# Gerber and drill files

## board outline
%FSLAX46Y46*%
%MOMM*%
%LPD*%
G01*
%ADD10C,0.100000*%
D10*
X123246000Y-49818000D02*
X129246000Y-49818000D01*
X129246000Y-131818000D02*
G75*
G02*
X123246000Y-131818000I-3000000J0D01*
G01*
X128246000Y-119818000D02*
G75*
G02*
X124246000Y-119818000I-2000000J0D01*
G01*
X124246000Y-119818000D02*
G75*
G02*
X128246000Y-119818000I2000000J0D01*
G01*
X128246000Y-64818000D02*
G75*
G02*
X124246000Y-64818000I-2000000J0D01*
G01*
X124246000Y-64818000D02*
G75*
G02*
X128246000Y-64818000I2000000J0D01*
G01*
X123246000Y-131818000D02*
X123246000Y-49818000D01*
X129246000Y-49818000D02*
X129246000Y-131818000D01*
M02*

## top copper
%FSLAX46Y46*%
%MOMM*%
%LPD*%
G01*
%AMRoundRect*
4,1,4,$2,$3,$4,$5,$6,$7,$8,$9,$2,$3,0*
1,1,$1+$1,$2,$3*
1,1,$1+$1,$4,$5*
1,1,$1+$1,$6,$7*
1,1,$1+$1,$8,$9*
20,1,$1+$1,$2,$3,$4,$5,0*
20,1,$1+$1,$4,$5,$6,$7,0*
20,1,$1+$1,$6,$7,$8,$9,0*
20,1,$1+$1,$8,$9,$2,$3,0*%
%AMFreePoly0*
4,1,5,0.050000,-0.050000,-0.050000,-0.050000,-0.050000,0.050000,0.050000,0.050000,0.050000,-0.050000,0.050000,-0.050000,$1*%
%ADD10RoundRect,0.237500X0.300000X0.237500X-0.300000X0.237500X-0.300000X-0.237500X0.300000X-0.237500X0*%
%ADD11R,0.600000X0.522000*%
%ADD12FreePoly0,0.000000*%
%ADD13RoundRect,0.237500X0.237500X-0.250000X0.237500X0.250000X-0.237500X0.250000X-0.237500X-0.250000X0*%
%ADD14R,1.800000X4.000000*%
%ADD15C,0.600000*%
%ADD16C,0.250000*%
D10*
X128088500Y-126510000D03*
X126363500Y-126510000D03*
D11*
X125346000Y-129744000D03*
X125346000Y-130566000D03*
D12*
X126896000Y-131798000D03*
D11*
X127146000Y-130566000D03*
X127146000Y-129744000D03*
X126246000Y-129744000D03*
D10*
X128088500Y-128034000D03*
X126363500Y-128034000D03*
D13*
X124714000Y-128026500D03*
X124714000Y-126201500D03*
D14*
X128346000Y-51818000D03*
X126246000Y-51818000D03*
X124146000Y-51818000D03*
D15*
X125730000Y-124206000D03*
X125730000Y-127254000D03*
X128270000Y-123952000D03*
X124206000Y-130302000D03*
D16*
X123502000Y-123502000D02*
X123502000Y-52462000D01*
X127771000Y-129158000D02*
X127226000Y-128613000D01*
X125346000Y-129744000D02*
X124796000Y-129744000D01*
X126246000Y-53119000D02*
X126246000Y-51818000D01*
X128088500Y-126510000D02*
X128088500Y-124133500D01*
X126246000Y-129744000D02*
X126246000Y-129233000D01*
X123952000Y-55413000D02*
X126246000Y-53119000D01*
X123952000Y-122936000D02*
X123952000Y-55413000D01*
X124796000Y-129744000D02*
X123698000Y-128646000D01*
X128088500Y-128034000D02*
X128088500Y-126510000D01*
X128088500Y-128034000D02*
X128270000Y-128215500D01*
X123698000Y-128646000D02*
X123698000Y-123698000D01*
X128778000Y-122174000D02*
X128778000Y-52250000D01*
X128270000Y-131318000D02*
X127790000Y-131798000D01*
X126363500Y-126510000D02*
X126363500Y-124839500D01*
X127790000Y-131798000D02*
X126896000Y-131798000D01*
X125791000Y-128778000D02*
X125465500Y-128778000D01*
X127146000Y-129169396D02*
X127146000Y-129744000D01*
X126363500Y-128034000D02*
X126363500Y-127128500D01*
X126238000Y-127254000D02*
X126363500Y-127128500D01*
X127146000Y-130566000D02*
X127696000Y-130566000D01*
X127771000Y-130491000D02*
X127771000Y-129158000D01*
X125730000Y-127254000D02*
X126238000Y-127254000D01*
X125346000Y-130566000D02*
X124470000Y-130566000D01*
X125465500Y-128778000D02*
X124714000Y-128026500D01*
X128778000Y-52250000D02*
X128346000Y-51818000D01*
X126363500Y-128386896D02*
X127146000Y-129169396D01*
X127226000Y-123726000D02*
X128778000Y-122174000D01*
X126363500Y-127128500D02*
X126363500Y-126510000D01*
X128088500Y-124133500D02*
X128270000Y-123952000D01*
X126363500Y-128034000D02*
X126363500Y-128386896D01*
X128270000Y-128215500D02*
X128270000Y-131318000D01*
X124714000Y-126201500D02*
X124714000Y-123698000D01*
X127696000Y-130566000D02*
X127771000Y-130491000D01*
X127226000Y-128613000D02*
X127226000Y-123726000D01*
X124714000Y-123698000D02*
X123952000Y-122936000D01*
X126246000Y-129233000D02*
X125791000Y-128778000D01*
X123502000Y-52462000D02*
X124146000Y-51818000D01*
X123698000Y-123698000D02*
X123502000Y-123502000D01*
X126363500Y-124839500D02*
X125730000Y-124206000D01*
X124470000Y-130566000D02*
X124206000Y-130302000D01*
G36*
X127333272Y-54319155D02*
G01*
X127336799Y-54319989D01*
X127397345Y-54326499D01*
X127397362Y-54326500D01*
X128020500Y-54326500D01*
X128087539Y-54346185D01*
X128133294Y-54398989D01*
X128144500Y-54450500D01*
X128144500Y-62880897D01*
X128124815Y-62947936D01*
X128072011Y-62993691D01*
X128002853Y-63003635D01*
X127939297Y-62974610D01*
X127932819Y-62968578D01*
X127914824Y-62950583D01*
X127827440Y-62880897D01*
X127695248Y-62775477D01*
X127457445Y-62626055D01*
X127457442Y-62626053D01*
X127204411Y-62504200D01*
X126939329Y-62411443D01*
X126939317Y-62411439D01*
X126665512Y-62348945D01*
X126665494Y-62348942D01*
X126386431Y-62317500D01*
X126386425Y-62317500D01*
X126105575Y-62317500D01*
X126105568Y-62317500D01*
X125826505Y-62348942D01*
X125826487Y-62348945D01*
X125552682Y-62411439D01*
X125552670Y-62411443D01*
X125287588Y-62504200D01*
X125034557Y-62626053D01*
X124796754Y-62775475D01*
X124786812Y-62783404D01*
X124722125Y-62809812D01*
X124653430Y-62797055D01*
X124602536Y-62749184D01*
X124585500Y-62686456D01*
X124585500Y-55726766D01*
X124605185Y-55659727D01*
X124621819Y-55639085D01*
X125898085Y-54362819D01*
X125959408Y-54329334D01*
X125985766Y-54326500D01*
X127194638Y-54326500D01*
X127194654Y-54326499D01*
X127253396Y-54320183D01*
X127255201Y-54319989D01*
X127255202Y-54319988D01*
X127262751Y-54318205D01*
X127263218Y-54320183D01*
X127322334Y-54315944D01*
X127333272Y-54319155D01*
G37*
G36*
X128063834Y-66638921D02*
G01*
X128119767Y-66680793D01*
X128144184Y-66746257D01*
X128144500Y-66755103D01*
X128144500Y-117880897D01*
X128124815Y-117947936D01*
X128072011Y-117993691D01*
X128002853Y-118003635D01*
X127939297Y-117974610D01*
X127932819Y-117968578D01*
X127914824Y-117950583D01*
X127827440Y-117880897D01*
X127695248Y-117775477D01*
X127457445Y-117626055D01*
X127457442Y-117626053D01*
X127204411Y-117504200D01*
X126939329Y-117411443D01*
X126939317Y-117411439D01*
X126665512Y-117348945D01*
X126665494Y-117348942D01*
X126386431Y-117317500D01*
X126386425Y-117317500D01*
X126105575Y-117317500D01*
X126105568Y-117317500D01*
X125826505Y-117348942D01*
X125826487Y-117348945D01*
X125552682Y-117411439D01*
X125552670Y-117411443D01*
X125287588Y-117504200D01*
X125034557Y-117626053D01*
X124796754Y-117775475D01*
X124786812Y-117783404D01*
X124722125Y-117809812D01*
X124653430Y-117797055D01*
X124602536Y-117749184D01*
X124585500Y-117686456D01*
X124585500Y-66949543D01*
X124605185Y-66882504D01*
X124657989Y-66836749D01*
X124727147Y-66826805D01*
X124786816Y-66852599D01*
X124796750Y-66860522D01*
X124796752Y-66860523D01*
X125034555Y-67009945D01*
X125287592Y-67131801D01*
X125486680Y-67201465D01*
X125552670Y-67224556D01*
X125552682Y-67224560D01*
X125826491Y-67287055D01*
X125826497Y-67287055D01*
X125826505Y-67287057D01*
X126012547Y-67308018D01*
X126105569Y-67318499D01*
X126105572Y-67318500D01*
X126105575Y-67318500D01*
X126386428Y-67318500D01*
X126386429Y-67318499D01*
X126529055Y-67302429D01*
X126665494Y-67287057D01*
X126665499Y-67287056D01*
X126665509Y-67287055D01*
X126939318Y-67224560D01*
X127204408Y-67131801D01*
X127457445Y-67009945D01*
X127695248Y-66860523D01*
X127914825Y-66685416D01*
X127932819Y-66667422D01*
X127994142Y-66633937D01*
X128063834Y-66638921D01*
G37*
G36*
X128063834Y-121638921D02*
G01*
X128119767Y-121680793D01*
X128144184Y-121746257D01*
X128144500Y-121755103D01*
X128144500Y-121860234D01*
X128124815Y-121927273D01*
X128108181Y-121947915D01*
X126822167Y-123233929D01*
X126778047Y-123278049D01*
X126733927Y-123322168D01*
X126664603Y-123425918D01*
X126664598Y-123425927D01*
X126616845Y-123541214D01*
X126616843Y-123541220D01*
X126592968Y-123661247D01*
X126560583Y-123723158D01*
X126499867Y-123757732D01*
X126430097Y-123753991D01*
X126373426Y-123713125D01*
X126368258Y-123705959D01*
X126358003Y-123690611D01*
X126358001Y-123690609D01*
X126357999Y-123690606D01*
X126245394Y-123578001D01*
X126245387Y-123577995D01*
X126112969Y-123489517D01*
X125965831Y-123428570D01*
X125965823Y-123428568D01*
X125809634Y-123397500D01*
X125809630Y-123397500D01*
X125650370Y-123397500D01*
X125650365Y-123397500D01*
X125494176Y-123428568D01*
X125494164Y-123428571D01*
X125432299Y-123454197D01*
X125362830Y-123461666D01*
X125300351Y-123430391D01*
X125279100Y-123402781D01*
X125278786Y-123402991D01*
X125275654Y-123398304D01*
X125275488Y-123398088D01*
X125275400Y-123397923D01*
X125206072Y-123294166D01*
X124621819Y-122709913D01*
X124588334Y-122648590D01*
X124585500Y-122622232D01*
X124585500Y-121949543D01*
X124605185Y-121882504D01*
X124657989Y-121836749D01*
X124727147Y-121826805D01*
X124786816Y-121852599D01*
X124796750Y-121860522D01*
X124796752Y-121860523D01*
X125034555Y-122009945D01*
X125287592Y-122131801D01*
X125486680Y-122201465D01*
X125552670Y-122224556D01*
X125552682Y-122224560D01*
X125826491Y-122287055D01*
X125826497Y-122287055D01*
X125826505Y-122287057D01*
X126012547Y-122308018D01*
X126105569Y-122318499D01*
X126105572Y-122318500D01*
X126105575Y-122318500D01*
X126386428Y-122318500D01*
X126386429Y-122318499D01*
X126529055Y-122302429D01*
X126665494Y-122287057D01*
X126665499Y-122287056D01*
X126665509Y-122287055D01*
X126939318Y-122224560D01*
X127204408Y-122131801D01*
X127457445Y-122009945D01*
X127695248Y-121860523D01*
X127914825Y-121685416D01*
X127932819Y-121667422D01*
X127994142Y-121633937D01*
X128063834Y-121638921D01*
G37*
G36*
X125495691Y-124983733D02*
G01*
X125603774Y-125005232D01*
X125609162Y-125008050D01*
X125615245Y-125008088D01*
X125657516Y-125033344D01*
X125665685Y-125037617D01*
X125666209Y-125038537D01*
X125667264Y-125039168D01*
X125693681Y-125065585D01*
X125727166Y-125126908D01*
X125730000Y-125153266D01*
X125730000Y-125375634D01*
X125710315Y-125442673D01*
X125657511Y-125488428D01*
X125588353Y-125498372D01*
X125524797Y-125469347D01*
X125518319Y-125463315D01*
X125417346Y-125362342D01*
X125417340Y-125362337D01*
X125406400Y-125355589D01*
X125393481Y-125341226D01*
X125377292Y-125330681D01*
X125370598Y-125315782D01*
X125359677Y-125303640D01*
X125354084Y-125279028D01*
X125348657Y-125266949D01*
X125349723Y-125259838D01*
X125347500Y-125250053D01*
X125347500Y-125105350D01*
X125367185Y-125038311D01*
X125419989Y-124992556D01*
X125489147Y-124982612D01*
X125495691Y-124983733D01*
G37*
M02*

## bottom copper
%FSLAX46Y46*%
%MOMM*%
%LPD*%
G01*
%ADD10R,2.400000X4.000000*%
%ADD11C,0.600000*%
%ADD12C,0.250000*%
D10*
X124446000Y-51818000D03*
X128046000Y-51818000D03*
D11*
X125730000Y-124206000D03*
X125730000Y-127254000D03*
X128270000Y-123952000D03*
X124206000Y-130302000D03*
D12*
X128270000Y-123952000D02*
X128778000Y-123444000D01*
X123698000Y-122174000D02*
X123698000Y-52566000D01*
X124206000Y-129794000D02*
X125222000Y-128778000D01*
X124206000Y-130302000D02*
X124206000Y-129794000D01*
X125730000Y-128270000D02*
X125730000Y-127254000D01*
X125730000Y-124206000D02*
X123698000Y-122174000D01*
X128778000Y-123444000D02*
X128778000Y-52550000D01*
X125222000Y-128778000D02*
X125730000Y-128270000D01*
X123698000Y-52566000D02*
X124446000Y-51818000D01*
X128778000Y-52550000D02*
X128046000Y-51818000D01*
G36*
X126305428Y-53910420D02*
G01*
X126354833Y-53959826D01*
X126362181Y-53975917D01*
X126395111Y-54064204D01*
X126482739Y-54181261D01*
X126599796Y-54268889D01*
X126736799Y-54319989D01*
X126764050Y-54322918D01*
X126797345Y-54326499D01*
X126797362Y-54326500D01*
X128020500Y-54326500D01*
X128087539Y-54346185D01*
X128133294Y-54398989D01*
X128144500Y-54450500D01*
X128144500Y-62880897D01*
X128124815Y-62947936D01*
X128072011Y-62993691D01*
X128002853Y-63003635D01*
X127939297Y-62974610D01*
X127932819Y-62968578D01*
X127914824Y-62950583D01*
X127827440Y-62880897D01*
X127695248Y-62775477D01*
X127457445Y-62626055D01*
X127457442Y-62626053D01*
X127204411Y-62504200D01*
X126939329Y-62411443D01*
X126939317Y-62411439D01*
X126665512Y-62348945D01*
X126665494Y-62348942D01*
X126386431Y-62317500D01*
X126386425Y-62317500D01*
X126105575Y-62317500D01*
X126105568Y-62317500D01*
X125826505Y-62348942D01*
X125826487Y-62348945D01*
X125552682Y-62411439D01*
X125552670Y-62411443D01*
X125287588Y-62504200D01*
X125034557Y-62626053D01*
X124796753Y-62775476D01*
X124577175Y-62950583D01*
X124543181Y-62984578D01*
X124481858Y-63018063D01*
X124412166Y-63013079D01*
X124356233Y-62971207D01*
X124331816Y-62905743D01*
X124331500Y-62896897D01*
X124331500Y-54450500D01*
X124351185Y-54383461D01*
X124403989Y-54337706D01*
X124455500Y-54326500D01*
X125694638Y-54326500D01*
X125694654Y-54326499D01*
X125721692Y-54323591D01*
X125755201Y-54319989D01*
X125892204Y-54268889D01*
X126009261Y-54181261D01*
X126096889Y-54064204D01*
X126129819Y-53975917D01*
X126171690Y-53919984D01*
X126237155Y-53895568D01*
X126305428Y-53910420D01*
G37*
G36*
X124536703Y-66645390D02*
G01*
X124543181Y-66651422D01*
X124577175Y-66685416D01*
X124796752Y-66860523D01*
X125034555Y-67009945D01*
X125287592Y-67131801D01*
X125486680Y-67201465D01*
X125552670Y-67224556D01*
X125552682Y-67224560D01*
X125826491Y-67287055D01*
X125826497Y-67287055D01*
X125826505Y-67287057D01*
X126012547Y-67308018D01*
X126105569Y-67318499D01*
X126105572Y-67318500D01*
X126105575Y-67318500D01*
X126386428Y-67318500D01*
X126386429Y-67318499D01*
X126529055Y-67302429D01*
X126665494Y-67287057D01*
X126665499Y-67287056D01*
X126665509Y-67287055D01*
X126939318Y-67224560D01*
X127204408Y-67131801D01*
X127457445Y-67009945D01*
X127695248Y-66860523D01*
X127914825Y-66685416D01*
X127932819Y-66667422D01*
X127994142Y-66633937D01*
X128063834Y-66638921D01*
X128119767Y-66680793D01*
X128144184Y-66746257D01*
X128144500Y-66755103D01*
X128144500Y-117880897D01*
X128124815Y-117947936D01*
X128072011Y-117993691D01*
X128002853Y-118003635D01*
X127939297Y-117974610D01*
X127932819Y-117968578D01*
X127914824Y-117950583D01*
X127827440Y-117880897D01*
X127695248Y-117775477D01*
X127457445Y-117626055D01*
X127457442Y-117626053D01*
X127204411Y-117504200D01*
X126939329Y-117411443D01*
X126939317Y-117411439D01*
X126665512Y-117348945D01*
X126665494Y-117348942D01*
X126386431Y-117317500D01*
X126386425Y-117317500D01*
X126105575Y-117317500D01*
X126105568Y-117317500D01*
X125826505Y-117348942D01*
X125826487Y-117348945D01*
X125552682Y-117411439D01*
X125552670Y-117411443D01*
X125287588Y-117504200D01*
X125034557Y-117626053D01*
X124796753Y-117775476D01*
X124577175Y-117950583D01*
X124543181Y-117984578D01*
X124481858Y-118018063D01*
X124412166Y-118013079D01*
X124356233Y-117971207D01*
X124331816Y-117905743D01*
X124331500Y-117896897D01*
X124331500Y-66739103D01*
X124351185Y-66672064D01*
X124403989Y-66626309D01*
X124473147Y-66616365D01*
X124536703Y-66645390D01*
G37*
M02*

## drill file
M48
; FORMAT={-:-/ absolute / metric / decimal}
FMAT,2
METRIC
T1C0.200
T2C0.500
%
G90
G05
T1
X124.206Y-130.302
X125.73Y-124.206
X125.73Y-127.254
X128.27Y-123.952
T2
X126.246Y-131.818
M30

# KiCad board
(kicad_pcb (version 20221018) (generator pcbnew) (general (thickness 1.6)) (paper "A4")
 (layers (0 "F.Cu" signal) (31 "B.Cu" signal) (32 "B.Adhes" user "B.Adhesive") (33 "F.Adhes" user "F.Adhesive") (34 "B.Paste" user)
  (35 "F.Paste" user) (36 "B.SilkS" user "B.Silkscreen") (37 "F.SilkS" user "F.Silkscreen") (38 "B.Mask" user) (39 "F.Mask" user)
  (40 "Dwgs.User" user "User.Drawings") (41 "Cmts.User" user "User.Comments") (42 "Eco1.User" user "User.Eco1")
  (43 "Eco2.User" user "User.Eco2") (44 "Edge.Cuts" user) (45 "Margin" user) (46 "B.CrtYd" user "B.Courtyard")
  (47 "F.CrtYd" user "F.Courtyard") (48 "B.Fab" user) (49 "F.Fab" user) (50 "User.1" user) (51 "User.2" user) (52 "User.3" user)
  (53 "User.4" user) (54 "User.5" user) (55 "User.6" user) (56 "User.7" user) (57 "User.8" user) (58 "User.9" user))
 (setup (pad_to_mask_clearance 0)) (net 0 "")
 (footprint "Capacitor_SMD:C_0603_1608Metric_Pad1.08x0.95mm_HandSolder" (layer "F.Cu") (at 127.226 126.51 180)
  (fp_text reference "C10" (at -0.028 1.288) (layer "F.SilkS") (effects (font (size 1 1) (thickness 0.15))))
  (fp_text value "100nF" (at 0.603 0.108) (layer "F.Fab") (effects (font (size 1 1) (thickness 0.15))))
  (pad "1" smd roundrect (at -0.8625 0 180) (size 1.075 0.95) (layers "F.Cu" "F.Paste" "F.Mask") (roundrect_rratio 0.25))
  (pad "2" smd roundrect (at 0.8625 0 180) (size 1.075 0.95) (layers "F.Cu" "F.Paste" "F.Mask") (roundrect_rratio 0.25)))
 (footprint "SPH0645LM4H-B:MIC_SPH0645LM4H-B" (layer "F.Cu") (at 126.246 131.818)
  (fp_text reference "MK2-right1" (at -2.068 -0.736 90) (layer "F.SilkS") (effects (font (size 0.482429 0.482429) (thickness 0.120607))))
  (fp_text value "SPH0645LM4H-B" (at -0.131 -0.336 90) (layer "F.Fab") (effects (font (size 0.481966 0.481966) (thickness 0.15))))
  (pad "" np_thru_hole circle (at 0 0) (size 0.5 0.5) (drill 0.5) (layers "*.Cu" "*.Mask"))
  (pad "1" smd rect (at -0.9 -2.074) (size 0.6 0.522) (layers "F.Cu" "F.Paste" "F.Mask"))
  (pad "2" smd rect (at -0.9 -1.252) (size 0.6 0.522) (layers "F.Cu" "F.Paste" "F.Mask"))
  (pad "3" smd custom (at 0.65 -0.02) (size 0.1 0.1) (layers "F.Cu") (zone_connect 0) (thermal_bridge_angle 45)
   (options (clearance outline) (anchor rect)) (primitives))
  (pad "4" smd rect (at 0.9 -1.252) (size 0.6 0.522) (layers "F.Cu" "F.Paste" "F.Mask"))
  (pad "5" smd rect (at 0.9 -2.074) (size 0.6 0.522) (layers "F.Cu" "F.Paste" "F.Mask"))
  (pad "6" smd rect (at 0 -2.074) (size 0.6 0.522) (layers "F.Cu" "F.Paste" "F.Mask")))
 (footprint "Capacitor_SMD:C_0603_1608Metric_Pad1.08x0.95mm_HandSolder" (layer "F.Cu") (at 127.226 128.034 180)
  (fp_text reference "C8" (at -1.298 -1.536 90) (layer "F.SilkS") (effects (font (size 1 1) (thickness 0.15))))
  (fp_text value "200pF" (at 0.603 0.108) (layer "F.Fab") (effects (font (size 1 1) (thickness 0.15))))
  (pad "1" smd roundrect (at -0.8625 0 180) (size 1.075 0.95) (layers "F.Cu" "F.Paste" "F.Mask") (roundrect_rratio 0.25))
  (pad "2" smd roundrect (at 0.8625 0 180) (size 1.075 0.95) (layers "F.Cu" "F.Paste" "F.Mask") (roundrect_rratio 0.25)))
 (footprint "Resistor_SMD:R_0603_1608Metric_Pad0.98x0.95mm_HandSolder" (layer "F.Cu") (at 124.714 127.114 90)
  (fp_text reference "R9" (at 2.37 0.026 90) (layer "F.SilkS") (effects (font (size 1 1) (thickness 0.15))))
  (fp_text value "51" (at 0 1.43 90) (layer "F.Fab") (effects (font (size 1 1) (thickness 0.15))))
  (pad "1" smd roundrect (at -0.9125 0 90) (size 0.975 0.95) (layers "F.Cu" "F.Paste" "F.Mask") (roundrect_rratio 0.25))
  (pad "2" smd roundrect (at 0.9125 0 90) (size 0.975 0.95) (layers "F.Cu" "F.Paste" "F.Mask") (roundrect_rratio 0.25)))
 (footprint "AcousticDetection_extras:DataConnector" (layer "F.Cu") (at 126.246 51.818 -90)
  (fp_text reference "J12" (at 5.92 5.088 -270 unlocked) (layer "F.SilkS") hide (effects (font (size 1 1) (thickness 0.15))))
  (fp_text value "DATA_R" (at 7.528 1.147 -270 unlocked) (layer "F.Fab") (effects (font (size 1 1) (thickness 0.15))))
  (pad "1" smd rect (at 0 -2.1 270) (size 4 1.8) (layers "F.Cu" "F.Paste" "F.Mask") (thermal_bridge_angle 45))
  (pad "2" smd rect (at 0 0 270) (size 4 1.8) (layers "F.Cu" "F.Paste" "F.Mask") (thermal_bridge_angle 45))
  (pad "3" smd rect (at 0 2.1 270) (size 4 1.8) (layers "F.Cu" "F.Paste" "F.Mask") (thermal_bridge_angle 45)))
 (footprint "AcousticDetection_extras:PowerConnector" (layer "B.Cu") (at 126.246 51.818 -90)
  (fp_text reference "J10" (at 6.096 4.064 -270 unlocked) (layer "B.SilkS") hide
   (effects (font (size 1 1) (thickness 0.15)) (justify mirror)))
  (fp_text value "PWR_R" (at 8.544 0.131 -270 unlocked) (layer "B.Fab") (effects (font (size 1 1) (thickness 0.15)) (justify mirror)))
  (pad "1" smd rect (at 0 1.8 270) (size 4 2.4) (layers "B.Cu" "B.Paste" "B.Mask") (thermal_bridge_angle 45))
  (pad "2" smd rect (at 0 -1.8 270) (size 4 2.4) (layers "B.Cu" "B.Paste" "B.Mask") (thermal_bridge_angle 45)))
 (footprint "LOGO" (layer "B.Cu") (at 126.238 132.08 -90)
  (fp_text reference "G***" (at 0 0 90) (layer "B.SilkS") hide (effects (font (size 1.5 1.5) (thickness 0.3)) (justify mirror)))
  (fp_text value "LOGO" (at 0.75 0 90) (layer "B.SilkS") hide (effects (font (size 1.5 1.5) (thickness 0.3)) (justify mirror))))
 (gr_line (start 123.246 49.818) (end 129.246 49.818) (stroke (width 0.1) (type solid)) (layer "Edge.Cuts"))
 (gr_arc (start 129.246 131.818) (mid 126.246 134.818) (end 123.246 131.818) (stroke (width 0.1) (type solid)) (layer "Edge.Cuts"))
 (gr_circle (center 126.246 119.818) (end 126.246 117.818) (stroke (width 0.1) (type default)) (fill none) (layer "Edge.Cuts"))
 (gr_circle (center 126.246 64.818) (end 126.246 62.818) (stroke (width 0.1) (type default)) (fill none) (layer "Edge.Cuts"))
 (gr_line (start 123.246 131.818) (end 123.246 49.818) (stroke (width 0.1) (type solid)) (layer "Edge.Cuts"))
 (gr_line (start 129.246 49.818) (end 129.246 131.818) (stroke (width 0.1) (type solid)) (layer "Edge.Cuts"))
 (segment (start 123.502 123.502) (end 123.502 52.462) (width 0.25) (layer "F.Cu") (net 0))
 (segment (start 127.771 129.158) (end 127.226 128.613) (width 0.25) (layer "F.Cu") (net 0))
 (segment (start 125.346 129.744) (end 124.796 129.744) (width 0.25) (layer "F.Cu") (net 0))
 (segment (start 126.246 53.119) (end 126.246 51.818) (width 0.25) (layer "F.Cu") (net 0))
 (segment (start 128.0885 126.51) (end 128.0885 124.1335) (width 0.25) (layer "F.Cu") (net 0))
 (segment (start 126.246 129.744) (end 126.246 129.233) (width 0.25) (layer "F.Cu") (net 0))
 (segment (start 123.952 55.413) (end 126.246 53.119) (width 0.25) (layer "F.Cu") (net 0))
 (segment (start 123.952 122.936) (end 123.952 55.413) (width 0.25) (layer "F.Cu") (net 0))
 (segment (start 124.796 129.744) (end 123.698 128.646) (width 0.25) (layer "F.Cu") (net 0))
 (segment (start 128.0885 128.034) (end 128.0885 126.51) (width 0.25) (layer "F.Cu") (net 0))
 (segment (start 128.0885 128.034) (end 128.27 128.2155) (width 0.25) (layer "F.Cu") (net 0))
 (segment (start 123.698 128.646) (end 123.698 123.698) (width 0.25) (layer "F.Cu") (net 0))
 (segment (start 128.778 122.174) (end 128.778 52.25) (width 0.25) (layer "F.Cu") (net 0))
 (segment (start 128.27 131.318) (end 127.79 131.798) (width 0.25) (layer "F.Cu") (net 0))
 (segment (start 126.3635 126.51) (end 126.3635 124.8395) (width 0.25) (layer "F.Cu") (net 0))
 (segment (start 127.79 131.798) (end 126.896 131.798) (width 0.25) (layer "F.Cu") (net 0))
 (segment (start 125.791 128.778) (end 125.4655 128.778) (width 0.25) (layer "F.Cu") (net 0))
 (segment (start 127.146 129.169396) (end 127.146 129.744) (width 0.25) (layer "F.Cu") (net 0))
 (segment (start 126.3635 128.034) (end 126.3635 127.1285) (width 0.25) (layer "F.Cu") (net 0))
 (segment (start 126.238 127.254) (end 126.3635 127.1285) (width 0.25) (layer "F.Cu") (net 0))
 (segment (start 127.146 130.566) (end 127.696 130.566) (width 0.25) (layer "F.Cu") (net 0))
 (segment (start 127.771 130.491) (end 127.771 129.158) (width 0.25) (layer "F.Cu") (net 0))
 (segment (start 125.73 127.254) (end 126.238 127.254) (width 0.25) (layer "F.Cu") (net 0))
 (segment (start 125.346 130.566) (end 124.47 130.566) (width 0.25) (layer "F.Cu") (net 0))
 (segment (start 125.4655 128.778) (end 124.714 128.0265) (width 0.25) (layer "F.Cu") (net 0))
 (segment (start 128.778 52.25) (end 128.346 51.818) (width 0.25) (layer "F.Cu") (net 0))
 (segment (start 126.3635 128.386896) (end 127.146 129.169396) (width 0.25) (layer "F.Cu") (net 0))
 (segment (start 127.226 123.726) (end 128.778 122.174) (width 0.25) (layer "F.Cu") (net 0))
 (segment (start 126.3635 127.1285) (end 126.3635 126.51) (width 0.25) (layer "F.Cu") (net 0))
 (segment (start 128.0885 124.1335) (end 128.27 123.952) (width 0.25) (layer "F.Cu") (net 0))
 (segment (start 126.3635 128.034) (end 126.3635 128.386896) (width 0.25) (layer "F.Cu") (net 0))
 (segment (start 128.27 128.2155) (end 128.27 131.318) (width 0.25) (layer "F.Cu") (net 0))
 (segment (start 124.714 126.2015) (end 124.714 123.698) (width 0.25) (layer "F.Cu") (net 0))
 (segment (start 127.696 130.566) (end 127.771 130.491) (width 0.25) (layer "F.Cu") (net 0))
 (segment (start 127.226 128.613) (end 127.226 123.726) (width 0.25) (layer "F.Cu") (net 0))
 (segment (start 124.714 123.698) (end 123.952 122.936) (width 0.25) (layer "F.Cu") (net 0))
 (segment (start 126.246 129.233) (end 125.791 128.778) (width 0.25) (layer "F.Cu") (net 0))
 (segment (start 123.502 52.462) (end 124.146 51.818) (width 0.25) (layer "F.Cu") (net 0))
 (segment (start 123.698 123.698) (end 123.502 123.502) (width 0.25) (layer "F.Cu") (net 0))
 (segment (start 126.3635 124.8395) (end 125.73 124.206) (width 0.25) (layer "F.Cu") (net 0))
 (segment (start 124.47 130.566) (end 124.206 130.302) (width 0.25) (layer "F.Cu") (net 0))
 (via (at 125.73 124.206) (size 0.6) (drill 0.2) (layers "F.Cu" "B.Cu") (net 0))
 (via (at 125.73 127.254) (size 0.6) (drill 0.2) (layers "F.Cu" "B.Cu") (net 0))
 (via (at 128.27 123.952) (size 0.6) (drill 0.2) (layers "F.Cu" "B.Cu") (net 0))
 (via (at 124.206 130.302) (size 0.6) (drill 0.2) (layers "F.Cu" "B.Cu") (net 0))
 (segment (start 128.27 123.952) (end 128.778 123.444) (width 0.25) (layer "B.Cu") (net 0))
 (segment (start 123.698 122.174) (end 123.698 52.566) (width 0.25) (layer "B.Cu") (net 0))
 (segment (start 124.206 129.794) (end 125.222 128.778) (width 0.25) (layer "B.Cu") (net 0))
 (segment (start 124.206 130.302) (end 124.206 129.794) (width 0.25) (layer "B.Cu") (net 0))
 (segment (start 125.73 128.27) (end 125.73 127.254) (width 0.25) (layer "B.Cu") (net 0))
 (segment (start 125.73 124.206) (end 123.698 122.174) (width 0.25) (layer "B.Cu") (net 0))
 (segment (start 128.778 123.444) (end 128.778 52.55) (width 0.25) (layer "B.Cu") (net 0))
 (segment (start 125.222 128.778) (end 125.73 128.27) (width 0.25) (layer "B.Cu") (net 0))
 (segment (start 123.698 52.566) (end 124.446 51.818) (width 0.25) (layer "B.Cu") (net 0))
 (segment (start 128.778 52.55) (end 128.046 51.818) (width 0.25) (layer "B.Cu") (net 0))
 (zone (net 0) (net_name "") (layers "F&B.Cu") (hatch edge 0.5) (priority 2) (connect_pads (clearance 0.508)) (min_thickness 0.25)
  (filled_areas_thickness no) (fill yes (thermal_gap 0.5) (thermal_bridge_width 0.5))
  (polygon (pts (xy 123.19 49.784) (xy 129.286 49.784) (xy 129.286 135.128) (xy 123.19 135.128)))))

